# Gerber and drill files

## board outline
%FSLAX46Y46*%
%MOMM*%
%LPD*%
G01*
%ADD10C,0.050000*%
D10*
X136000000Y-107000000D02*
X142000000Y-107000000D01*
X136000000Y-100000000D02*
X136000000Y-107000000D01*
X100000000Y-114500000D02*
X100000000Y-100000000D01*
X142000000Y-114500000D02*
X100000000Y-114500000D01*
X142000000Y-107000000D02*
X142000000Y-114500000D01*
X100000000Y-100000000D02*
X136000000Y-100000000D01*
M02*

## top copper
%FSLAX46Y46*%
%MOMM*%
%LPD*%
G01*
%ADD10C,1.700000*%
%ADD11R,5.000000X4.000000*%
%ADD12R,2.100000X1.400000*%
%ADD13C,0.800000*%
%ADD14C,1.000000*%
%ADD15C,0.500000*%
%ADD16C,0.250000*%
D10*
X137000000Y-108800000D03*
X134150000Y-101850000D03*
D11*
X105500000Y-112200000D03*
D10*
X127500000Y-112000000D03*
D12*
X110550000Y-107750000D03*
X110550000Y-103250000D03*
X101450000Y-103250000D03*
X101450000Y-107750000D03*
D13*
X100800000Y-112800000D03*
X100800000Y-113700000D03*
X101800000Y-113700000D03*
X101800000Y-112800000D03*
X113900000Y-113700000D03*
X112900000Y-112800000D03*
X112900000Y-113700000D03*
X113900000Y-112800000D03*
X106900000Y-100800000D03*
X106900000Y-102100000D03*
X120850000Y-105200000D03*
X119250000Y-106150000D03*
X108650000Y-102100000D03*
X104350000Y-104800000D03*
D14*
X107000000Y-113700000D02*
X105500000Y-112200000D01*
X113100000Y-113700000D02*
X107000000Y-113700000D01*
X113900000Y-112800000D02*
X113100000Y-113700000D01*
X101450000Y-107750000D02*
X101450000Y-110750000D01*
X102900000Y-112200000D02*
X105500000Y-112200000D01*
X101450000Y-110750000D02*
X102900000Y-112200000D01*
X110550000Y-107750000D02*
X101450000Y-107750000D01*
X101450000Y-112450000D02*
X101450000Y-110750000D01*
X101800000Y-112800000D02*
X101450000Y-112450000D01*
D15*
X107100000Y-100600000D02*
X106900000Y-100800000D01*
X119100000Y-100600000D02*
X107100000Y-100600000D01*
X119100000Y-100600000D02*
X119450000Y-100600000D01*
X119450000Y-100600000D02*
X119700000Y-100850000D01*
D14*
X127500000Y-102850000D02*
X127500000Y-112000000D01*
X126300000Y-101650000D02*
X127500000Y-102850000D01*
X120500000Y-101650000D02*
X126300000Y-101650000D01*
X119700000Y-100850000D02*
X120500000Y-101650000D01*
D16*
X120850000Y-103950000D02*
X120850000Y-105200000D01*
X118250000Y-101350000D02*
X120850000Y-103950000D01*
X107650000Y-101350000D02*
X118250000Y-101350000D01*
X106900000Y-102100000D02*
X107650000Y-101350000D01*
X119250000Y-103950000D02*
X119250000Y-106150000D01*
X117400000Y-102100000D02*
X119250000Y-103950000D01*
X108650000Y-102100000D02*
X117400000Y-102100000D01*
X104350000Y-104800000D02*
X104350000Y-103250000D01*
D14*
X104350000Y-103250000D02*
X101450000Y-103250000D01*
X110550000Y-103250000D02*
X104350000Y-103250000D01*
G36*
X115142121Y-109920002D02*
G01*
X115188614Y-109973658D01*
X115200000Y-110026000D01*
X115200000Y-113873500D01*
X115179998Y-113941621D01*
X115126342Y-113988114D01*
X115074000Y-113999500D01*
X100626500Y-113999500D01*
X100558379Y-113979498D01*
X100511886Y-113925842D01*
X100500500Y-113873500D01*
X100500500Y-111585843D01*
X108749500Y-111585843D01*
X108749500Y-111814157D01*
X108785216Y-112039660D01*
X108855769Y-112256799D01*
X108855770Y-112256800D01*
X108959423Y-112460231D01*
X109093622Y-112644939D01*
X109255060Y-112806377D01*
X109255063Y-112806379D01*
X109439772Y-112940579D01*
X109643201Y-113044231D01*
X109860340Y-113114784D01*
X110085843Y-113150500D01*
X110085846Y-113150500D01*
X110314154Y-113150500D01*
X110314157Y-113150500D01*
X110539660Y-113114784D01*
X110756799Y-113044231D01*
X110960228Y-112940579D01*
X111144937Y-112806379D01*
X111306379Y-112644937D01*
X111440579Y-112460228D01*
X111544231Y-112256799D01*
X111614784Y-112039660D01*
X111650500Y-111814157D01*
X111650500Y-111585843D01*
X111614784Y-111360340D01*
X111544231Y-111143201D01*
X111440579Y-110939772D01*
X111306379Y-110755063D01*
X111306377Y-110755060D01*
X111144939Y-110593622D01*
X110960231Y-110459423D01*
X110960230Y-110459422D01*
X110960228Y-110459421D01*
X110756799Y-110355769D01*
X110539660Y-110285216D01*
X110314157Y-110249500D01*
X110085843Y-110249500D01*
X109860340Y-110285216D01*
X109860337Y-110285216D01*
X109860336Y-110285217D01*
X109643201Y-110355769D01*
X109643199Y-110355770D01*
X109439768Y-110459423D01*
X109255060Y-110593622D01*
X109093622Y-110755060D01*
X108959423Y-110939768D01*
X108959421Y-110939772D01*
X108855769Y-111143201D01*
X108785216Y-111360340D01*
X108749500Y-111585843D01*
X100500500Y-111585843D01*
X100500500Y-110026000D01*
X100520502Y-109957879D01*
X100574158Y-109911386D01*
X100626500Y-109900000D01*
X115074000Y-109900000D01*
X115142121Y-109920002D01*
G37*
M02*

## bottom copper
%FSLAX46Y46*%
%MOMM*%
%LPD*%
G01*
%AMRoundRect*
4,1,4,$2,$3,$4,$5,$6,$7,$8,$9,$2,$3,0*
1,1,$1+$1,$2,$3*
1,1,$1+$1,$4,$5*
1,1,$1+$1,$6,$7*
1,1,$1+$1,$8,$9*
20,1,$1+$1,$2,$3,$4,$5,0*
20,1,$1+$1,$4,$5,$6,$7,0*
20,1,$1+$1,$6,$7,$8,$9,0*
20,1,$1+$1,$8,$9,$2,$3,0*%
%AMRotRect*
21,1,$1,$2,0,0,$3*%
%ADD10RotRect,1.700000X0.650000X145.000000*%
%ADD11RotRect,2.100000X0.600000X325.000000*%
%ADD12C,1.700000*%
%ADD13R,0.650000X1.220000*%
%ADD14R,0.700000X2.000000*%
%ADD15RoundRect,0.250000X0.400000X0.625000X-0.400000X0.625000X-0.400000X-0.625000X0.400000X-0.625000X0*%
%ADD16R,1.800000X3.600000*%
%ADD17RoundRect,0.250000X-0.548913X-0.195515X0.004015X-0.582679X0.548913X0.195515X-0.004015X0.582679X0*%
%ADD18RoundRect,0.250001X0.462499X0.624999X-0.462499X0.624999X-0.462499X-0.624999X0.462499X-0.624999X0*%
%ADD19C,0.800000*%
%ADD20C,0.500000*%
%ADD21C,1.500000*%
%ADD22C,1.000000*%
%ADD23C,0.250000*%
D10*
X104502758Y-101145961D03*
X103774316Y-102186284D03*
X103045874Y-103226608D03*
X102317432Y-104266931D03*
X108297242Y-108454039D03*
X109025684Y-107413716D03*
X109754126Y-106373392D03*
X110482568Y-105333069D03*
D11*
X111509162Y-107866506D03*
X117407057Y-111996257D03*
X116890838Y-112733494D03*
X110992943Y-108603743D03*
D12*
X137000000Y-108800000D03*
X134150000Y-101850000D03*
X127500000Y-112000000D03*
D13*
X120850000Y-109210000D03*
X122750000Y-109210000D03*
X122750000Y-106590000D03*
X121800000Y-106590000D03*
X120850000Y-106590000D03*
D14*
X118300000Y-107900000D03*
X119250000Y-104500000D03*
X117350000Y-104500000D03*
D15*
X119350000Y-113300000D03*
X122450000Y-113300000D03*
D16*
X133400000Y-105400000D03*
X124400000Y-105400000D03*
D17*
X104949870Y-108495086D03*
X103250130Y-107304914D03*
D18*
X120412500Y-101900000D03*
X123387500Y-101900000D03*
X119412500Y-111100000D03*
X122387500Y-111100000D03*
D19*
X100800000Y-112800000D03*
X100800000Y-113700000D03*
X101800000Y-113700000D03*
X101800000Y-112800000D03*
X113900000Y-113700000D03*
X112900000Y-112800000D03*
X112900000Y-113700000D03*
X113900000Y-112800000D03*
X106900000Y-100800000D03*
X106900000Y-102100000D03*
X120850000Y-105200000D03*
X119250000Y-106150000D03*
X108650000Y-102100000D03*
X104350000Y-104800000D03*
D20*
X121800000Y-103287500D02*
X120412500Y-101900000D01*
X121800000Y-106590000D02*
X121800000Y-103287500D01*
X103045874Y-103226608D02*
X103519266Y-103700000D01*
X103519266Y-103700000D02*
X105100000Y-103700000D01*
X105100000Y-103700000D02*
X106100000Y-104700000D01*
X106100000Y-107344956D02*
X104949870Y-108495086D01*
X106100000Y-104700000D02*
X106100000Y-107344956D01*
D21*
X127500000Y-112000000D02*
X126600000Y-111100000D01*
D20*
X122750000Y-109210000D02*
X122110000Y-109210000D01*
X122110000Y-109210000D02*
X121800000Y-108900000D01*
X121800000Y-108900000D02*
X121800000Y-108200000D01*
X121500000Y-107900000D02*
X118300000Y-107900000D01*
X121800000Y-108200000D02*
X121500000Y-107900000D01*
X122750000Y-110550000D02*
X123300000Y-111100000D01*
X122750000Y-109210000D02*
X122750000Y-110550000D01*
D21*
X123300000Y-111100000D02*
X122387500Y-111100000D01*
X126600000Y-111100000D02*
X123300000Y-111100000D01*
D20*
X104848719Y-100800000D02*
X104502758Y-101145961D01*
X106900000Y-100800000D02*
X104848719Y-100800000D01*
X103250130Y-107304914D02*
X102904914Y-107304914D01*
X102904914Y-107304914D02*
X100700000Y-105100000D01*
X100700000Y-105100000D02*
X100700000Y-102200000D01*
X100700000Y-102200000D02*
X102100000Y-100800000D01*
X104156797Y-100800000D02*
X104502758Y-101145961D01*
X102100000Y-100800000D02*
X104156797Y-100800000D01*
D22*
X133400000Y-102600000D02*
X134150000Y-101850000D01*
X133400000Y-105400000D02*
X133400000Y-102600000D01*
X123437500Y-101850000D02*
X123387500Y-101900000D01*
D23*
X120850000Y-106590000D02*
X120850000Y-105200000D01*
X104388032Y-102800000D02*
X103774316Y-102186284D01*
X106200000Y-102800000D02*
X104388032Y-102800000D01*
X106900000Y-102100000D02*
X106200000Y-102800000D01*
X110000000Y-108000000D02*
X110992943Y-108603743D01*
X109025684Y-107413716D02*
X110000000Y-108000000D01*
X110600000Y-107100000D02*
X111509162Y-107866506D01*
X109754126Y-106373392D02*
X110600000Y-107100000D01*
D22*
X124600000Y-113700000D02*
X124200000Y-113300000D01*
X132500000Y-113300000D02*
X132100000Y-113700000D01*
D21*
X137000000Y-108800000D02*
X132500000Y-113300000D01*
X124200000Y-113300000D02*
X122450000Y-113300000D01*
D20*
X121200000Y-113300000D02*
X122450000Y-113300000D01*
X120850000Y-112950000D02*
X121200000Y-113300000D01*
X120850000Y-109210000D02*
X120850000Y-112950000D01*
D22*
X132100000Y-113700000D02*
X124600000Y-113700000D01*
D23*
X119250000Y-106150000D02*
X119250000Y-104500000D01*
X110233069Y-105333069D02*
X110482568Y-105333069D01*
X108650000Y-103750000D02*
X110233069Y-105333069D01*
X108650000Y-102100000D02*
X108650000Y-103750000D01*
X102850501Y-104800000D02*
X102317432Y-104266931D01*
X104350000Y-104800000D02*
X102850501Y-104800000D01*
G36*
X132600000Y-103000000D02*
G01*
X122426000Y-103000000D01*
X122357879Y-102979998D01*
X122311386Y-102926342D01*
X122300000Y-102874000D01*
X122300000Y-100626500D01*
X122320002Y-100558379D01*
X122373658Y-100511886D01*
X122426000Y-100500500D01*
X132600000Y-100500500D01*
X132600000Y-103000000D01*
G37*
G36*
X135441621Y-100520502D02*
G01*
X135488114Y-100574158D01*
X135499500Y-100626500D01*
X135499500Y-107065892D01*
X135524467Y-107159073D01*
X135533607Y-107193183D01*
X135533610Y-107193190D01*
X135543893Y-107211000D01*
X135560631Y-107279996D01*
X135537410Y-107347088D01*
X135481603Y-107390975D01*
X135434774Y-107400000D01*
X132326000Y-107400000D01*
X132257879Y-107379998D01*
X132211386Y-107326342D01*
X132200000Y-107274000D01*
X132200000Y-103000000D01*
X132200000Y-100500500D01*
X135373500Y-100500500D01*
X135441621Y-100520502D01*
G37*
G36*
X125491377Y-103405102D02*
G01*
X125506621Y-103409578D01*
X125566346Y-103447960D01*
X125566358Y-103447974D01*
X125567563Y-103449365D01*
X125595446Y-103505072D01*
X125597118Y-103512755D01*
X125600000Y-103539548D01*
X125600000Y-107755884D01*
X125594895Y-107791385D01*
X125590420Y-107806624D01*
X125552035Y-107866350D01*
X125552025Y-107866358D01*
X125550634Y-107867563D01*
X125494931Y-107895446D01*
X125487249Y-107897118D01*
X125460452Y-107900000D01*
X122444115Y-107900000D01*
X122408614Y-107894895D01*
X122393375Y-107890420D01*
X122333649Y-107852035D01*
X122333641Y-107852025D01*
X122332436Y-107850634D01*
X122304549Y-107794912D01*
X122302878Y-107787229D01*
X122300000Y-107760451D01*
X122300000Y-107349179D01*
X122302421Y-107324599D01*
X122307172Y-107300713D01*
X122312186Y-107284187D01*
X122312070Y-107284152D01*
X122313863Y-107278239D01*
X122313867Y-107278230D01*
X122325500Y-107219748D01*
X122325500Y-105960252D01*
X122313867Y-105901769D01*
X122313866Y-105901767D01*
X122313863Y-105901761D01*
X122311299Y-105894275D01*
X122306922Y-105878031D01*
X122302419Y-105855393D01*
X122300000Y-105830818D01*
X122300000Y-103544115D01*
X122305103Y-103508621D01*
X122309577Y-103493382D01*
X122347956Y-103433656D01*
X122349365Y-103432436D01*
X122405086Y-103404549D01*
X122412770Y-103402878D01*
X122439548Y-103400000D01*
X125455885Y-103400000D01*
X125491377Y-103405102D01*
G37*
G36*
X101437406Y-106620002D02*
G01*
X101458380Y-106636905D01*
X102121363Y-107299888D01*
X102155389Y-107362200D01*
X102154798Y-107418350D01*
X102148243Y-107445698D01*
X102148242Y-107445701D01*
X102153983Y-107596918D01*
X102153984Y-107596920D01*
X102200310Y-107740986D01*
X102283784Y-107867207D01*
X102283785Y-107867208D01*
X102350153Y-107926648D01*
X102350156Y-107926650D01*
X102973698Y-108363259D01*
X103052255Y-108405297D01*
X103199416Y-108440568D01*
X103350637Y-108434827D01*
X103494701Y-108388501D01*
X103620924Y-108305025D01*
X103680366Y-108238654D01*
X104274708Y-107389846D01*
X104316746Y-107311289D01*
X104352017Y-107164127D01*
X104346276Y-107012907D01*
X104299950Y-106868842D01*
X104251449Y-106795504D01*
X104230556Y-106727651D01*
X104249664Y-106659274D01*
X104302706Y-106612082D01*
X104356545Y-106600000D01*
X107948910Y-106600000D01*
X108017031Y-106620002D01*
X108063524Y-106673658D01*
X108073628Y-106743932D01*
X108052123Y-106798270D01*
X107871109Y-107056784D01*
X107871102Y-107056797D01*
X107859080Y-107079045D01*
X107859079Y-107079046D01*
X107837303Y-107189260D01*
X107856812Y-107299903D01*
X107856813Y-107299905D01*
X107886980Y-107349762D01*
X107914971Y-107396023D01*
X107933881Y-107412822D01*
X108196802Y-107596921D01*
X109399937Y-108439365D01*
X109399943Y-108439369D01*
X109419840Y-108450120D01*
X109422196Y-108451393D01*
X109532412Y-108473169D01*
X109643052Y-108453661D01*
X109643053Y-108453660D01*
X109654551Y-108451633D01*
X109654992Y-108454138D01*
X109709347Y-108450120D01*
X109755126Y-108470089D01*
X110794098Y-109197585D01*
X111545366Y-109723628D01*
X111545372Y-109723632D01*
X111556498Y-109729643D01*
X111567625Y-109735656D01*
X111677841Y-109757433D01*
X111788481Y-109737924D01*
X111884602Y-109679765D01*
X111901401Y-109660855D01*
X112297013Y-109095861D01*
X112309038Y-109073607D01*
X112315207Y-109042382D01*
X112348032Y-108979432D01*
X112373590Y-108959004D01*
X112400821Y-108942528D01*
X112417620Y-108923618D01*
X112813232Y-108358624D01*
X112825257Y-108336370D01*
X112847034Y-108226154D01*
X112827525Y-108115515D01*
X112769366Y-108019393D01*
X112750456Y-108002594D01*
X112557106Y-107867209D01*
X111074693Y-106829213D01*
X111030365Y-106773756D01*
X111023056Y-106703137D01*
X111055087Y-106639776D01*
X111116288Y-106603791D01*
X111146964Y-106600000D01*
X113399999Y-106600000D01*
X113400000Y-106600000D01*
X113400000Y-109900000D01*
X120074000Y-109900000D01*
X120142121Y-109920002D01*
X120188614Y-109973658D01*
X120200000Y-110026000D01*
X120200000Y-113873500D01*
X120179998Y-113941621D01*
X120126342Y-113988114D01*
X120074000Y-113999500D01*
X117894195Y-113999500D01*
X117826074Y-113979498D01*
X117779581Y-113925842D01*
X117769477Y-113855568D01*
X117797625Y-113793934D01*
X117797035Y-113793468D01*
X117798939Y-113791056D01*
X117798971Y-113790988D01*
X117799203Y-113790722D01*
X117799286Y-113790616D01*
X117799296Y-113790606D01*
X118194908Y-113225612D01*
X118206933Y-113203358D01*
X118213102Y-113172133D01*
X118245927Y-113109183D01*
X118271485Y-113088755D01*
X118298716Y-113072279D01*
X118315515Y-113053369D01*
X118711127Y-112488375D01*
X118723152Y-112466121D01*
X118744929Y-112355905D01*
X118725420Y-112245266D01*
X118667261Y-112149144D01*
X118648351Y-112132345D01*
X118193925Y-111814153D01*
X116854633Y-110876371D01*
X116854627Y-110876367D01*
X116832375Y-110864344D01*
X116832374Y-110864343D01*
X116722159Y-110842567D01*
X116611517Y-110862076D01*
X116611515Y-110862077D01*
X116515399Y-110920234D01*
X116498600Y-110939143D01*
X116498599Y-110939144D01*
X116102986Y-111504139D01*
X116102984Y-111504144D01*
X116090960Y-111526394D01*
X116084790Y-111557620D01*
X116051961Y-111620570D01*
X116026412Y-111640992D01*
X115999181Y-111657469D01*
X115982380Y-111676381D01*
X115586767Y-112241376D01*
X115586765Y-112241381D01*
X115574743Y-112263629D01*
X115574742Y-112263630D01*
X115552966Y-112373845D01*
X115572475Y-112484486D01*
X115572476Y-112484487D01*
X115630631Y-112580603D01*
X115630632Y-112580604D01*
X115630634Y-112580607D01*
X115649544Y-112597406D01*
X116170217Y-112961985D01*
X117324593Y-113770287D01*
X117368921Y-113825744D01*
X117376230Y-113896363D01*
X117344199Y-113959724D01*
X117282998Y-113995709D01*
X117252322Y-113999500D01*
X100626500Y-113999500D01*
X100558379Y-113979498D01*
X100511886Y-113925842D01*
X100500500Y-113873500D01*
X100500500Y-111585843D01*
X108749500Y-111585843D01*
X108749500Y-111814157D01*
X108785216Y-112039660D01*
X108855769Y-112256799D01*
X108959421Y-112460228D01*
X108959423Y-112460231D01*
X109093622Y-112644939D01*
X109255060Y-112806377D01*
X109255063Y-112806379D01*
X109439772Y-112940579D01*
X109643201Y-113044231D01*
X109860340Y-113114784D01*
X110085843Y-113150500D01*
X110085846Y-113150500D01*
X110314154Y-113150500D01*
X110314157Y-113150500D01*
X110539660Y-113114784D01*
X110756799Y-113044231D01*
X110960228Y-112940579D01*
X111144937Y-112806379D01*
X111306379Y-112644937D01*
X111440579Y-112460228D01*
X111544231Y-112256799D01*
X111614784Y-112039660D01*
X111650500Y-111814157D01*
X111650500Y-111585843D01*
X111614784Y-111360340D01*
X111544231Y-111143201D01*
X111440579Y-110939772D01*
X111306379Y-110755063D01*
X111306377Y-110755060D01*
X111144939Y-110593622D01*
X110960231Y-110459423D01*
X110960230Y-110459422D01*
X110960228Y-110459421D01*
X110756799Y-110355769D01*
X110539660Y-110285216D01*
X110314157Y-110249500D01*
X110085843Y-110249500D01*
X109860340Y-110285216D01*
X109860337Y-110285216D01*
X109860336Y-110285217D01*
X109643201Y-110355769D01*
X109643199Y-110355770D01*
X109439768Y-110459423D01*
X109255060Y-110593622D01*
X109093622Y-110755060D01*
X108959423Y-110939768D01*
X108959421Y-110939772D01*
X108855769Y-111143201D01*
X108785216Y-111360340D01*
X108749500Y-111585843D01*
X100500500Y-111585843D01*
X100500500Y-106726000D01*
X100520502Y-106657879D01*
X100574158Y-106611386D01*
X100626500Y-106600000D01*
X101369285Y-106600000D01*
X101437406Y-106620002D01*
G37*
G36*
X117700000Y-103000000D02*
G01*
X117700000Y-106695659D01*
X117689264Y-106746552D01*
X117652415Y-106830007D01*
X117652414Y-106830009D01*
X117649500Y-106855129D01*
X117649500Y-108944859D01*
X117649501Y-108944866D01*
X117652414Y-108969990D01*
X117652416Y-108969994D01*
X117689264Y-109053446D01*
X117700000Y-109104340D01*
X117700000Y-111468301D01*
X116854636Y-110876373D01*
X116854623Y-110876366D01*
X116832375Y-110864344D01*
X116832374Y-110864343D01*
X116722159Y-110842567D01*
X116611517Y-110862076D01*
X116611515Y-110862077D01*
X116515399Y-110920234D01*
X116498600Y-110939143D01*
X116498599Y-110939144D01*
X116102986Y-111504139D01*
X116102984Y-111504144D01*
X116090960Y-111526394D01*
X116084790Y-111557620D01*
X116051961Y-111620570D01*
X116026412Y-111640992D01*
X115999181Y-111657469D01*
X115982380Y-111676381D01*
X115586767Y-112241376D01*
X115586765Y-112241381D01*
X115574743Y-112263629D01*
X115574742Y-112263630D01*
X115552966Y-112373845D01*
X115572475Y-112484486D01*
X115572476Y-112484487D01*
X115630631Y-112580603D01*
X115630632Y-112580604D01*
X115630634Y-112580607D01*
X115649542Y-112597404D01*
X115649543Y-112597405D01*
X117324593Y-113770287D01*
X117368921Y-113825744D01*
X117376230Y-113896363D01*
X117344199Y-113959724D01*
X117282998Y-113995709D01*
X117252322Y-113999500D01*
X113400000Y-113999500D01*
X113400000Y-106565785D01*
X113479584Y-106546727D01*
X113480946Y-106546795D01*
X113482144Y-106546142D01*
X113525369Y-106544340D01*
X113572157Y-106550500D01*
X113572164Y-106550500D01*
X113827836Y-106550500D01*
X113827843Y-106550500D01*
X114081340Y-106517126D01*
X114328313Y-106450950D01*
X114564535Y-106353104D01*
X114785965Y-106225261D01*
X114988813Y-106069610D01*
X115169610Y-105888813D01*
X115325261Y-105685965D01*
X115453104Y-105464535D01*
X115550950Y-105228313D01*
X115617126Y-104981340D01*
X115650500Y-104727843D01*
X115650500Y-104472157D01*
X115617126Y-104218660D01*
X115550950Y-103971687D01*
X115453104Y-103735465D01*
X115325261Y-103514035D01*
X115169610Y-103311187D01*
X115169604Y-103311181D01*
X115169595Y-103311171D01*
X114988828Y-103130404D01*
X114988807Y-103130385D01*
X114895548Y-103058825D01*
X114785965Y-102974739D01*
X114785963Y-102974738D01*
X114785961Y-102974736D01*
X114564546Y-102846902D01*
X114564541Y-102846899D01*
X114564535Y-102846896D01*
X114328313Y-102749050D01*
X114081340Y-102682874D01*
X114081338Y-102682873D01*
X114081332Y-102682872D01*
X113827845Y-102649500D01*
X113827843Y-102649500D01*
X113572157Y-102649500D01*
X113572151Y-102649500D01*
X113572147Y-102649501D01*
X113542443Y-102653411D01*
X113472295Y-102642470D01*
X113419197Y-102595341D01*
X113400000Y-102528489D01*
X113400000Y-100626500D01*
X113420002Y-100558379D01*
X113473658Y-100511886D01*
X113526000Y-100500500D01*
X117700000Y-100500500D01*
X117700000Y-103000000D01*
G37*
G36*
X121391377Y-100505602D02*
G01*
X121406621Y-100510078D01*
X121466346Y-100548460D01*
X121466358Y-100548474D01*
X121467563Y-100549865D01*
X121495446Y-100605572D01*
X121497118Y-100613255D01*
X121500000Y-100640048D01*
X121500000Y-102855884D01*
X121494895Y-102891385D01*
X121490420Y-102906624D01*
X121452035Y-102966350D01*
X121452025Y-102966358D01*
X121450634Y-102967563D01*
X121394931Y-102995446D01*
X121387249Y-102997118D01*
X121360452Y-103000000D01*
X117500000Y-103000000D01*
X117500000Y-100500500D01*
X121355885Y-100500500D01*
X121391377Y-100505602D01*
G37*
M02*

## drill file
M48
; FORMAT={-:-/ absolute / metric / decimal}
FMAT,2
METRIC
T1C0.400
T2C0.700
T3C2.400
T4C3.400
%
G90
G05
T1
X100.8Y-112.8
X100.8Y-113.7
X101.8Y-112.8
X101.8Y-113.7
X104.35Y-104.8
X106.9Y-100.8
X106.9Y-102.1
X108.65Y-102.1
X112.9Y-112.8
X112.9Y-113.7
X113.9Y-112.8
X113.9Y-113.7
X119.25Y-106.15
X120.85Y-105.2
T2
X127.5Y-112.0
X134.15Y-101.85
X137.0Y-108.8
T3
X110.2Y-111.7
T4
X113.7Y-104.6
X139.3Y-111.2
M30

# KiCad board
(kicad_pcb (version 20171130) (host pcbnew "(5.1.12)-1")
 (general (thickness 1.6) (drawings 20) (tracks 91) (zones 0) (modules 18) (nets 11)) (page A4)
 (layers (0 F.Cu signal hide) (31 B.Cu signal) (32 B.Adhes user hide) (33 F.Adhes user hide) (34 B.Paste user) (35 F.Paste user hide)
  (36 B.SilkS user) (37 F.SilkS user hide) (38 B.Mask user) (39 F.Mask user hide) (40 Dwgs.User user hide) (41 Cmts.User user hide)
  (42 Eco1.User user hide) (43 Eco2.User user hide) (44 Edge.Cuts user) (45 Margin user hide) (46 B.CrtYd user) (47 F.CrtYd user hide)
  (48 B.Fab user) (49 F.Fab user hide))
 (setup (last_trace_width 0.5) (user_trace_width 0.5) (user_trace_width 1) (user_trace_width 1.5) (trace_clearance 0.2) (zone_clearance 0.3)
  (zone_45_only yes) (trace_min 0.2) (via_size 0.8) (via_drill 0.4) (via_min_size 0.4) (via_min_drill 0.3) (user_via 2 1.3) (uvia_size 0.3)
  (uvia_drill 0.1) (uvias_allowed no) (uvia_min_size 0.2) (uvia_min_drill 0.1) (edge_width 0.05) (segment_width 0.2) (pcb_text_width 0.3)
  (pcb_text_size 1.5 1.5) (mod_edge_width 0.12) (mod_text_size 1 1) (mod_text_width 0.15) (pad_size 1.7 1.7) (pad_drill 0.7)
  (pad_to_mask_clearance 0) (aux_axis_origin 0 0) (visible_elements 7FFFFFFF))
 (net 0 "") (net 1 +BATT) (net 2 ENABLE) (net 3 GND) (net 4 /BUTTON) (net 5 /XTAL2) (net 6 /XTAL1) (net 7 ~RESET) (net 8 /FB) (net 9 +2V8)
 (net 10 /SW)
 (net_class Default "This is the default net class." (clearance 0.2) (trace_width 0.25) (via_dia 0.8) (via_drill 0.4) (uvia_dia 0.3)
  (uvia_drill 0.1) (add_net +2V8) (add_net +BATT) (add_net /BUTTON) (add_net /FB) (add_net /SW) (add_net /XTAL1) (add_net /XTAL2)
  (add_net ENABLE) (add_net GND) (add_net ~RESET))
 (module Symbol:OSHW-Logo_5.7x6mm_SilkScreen (layer F.Cu) (at 132.1 106.2)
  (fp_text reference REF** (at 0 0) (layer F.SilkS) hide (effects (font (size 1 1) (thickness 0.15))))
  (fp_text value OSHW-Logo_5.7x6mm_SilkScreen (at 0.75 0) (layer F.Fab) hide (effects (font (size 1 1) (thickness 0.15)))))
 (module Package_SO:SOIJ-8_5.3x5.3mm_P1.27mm (layer B.Cu) (at 106.4 104.8 145)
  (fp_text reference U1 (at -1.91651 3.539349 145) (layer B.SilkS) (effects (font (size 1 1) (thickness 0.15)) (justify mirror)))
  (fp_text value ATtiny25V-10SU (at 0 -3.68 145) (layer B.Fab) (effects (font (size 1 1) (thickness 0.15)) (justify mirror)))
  (pad 8 smd rect (at 3.65 1.905 145) (size 1.7 0.65) (layers B.Cu B.Paste B.Mask) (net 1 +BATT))
  (pad 7 smd rect (at 3.65 0.635 145) (size 1.7 0.65) (layers B.Cu B.Paste B.Mask) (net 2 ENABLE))
  (pad 6 smd rect (at 3.65 -0.635 145) (size 1.7 0.65) (layers B.Cu B.Paste B.Mask) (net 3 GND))
  (pad 5 smd rect (at 3.65 -1.905 145) (size 1.7 0.65) (layers B.Cu B.Paste B.Mask) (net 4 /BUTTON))
  (pad 4 smd rect (at -3.65 -1.905 145) (size 1.7 0.65) (layers B.Cu B.Paste B.Mask) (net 3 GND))
  (pad 3 smd rect (at -3.65 -0.635 145) (size 1.7 0.65) (layers B.Cu B.Paste B.Mask) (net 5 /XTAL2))
  (pad 2 smd rect (at -3.65 0.635 145) (size 1.7 0.65) (layers B.Cu B.Paste B.Mask) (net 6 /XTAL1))
  (pad 1 smd rect (at -3.65 1.905 145) (size 1.7 0.65) (layers B.Cu B.Paste B.Mask) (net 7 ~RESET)))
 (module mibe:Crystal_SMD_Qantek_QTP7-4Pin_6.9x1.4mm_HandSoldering (layer B.Cu) (at 114.2 110.3 325)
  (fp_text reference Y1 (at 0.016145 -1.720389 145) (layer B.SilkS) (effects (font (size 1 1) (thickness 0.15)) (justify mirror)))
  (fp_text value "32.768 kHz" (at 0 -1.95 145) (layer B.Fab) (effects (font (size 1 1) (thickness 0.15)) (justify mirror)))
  (pad 1 smd rect (at -3.6 -0.45 325) (size 2.1 0.6) (layers B.Cu B.Paste B.Mask) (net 6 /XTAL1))
  (pad NC smd rect (at 3.6 -0.45 325) (size 2.1 0.6) (layers B.Cu B.Paste B.Mask))
  (pad NC smd rect (at 3.6 0.45 325) (size 2.1 0.6) (layers B.Cu B.Paste B.Mask))
  (pad 2 smd rect (at -3.6 0.45 325) (size 2.1 0.6) (layers B.Cu B.Paste B.Mask) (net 5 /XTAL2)))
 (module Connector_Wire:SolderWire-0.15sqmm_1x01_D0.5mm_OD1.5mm (layer F.Cu) (at 137 108.8)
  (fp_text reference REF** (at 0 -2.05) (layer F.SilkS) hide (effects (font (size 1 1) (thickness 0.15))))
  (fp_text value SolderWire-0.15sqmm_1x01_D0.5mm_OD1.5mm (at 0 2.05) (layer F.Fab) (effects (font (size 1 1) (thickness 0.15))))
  (pad 1 thru_hole circle (at 0 0) (size 1.7 1.7) (drill 0.7) (layers *.Cu *.Mask) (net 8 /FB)))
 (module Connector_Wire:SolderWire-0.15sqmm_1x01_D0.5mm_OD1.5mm (layer F.Cu) (at 134.15 101.85)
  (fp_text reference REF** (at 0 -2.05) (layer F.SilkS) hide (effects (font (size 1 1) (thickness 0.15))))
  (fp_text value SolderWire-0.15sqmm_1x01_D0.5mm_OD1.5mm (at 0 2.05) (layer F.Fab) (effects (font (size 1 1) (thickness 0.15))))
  (pad 1 thru_hole circle (at 0 0) (size 1.7 1.7) (drill 0.7) (layers *.Cu *.Mask) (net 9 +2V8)))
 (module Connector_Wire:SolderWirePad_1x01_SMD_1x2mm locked (layer F.Cu) (at 105.5 112.2)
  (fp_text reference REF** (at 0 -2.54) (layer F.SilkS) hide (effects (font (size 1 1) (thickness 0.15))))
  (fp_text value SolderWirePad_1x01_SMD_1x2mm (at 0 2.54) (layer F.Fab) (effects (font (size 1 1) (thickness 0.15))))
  (pad 1 smd rect (at 0 0) (size 5 4) (layers F.Cu F.Paste F.Mask) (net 3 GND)))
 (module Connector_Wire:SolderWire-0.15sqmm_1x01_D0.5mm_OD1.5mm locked (layer F.Cu) (at 127.5 112)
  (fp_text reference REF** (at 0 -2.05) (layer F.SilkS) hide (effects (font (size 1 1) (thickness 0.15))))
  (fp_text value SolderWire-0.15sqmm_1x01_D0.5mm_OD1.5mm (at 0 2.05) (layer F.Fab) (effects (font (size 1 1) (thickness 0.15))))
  (pad 1 thru_hole circle (at 0 0) (size 1.7 1.7) (drill 0.7) (layers *.Cu *.Mask) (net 1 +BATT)))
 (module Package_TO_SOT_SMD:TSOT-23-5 (layer B.Cu) (at 121.8 107.9 270)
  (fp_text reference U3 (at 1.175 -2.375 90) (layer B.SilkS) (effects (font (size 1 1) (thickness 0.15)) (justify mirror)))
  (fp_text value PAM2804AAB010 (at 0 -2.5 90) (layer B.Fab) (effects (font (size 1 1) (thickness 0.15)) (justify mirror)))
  (pad 5 smd rect (at 1.31 0.95 270) (size 1.22 0.65) (layers B.Cu B.Paste B.Mask) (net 8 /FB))
  (pad 4 smd rect (at 1.31 -0.95 270) (size 1.22 0.65) (layers B.Cu B.Paste B.Mask) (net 1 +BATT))
  (pad 3 smd rect (at -1.31 -0.95 270) (size 1.22 0.65) (layers B.Cu B.Paste B.Mask) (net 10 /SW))
  (pad 2 smd rect (at -1.31 0 270) (size 1.22 0.65) (layers B.Cu B.Paste B.Mask) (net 3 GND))
  (pad 1 smd rect (at -1.31 0.95 270) (size 1.22 0.65) (layers B.Cu B.Paste B.Mask) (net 2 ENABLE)))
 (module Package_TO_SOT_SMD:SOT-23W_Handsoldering (layer B.Cu) (at 118.3 106.2 270)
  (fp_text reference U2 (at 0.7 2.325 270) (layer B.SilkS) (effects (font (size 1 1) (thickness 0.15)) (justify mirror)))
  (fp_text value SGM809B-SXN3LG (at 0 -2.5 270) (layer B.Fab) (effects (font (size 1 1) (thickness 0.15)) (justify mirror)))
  (pad 3 smd rect (at 1.7 0 270) (size 2 0.7) (layers B.Cu B.Paste B.Mask) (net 1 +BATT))
  (pad 2 smd rect (at -1.7 -0.95 270) (size 2 0.7) (layers B.Cu B.Paste B.Mask) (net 7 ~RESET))
  (pad 1 smd rect (at -1.7 0.95 270) (size 2 0.7) (layers B.Cu B.Paste B.Mask) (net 3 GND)))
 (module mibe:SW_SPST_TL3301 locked (layer F.Cu) (at 106 105.5)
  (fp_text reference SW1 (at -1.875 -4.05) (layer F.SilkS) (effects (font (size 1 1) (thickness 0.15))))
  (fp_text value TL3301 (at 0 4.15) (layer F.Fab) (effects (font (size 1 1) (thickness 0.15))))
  (pad 2 smd rect (at 4.55 2.25) (size 2.1 1.4) (layers F.Cu F.Paste F.Mask) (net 3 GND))
  (pad 1 smd rect (at 4.55 -2.25) (size 2.1 1.4) (layers F.Cu F.Paste F.Mask) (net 4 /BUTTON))
  (pad 1 smd rect (at -4.55 -2.25) (size 2.1 1.4) (layers F.Cu F.Paste F.Mask) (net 4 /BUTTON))
  (pad 2 smd rect (at -4.55 2.25) (size 2.1 1.4) (layers F.Cu F.Paste F.Mask) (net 3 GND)))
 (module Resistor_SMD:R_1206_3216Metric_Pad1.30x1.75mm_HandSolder (layer B.Cu) (at 120.9 113.3 180)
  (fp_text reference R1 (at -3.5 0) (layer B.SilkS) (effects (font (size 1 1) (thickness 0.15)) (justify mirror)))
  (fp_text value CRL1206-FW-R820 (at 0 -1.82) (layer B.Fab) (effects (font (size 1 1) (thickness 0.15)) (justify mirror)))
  (pad 2 smd roundrect (at 1.55 0 180) (size 1.3 1.75) (layers B.Cu B.Paste B.Mask) (roundrect_rratio 0.192308) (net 3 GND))
  (pad 1 smd roundrect (at -1.55 0 180) (size 1.3 1.75) (layers B.Cu B.Paste B.Mask) (roundrect_rratio 0.192308) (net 8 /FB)))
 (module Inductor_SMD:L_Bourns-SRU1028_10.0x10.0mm (layer B.Cu) (at 128.9 105.4)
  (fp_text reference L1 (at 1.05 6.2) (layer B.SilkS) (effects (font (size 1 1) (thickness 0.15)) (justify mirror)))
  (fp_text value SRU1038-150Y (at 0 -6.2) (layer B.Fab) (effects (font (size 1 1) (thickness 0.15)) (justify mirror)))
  (pad 2 smd rect (at 4.5 0) (size 1.8 3.6) (layers B.Cu B.Paste B.Mask) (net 9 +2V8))
  (pad 1 smd rect (at -4.5 0) (size 1.8 3.6) (layers B.Cu B.Paste B.Mask) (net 10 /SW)))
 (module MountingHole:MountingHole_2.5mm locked (layer F.Cu) (at 110.2 111.7)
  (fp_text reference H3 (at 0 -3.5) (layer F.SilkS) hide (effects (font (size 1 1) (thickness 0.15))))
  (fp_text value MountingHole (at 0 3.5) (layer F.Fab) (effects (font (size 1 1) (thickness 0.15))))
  (pad "" np_thru_hole circle (at 0 0) (size 2.4 2.4) (drill 2.4) (layers *.Cu *.Mask)))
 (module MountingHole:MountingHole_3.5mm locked (layer F.Cu) (at 139.3 111.2)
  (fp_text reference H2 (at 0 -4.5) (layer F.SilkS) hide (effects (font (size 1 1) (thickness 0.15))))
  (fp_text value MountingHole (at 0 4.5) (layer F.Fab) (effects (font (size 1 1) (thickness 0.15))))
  (pad "" np_thru_hole circle (at 0 0) (size 3.4 3.4) (drill 3.4) (layers *.Cu *.Mask)))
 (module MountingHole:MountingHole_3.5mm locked (layer F.Cu) (at 113.7 104.6)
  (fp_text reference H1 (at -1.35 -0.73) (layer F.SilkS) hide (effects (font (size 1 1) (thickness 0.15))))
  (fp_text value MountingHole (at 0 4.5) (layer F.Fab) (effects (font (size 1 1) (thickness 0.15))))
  (pad "" np_thru_hole circle (at 0 0) (size 3.4 3.4) (drill 3.4) (layers *.Cu *.Mask)))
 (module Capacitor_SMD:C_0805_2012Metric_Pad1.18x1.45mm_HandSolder (layer B.Cu) (at 104.1 107.9 325)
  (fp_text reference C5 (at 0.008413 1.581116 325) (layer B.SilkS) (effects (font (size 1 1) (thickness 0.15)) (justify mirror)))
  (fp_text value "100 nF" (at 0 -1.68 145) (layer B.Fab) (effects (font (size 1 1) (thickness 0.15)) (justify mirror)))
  (pad 2 smd roundrect (at 1.0375 0 325) (size 1.175 1.45) (layers B.Cu B.Paste B.Mask) (roundrect_rratio 0.212766) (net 3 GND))
  (pad 1 smd roundrect (at -1.0375 0 325) (size 1.175 1.45) (layers B.Cu B.Paste B.Mask) (roundrect_rratio 0.212766) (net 1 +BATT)))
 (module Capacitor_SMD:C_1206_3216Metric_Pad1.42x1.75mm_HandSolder (layer B.Cu) (at 121.9 101.9 180)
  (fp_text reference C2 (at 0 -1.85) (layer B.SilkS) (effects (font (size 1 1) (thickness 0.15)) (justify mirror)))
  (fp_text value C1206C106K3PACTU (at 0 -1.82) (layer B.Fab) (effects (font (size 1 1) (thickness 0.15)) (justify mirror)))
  (pad 2 smd roundrect (at 1.4875 0 180) (size 1.425 1.75) (layers B.Cu B.Paste B.Mask) (roundrect_rratio 0.175439) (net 3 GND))
  (pad 1 smd roundrect (at -1.4875 0 180) (size 1.425 1.75) (layers B.Cu B.Paste B.Mask) (roundrect_rratio 0.175439) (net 9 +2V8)))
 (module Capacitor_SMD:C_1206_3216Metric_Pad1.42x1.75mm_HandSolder (layer B.Cu) (at 120.9 111.1 180)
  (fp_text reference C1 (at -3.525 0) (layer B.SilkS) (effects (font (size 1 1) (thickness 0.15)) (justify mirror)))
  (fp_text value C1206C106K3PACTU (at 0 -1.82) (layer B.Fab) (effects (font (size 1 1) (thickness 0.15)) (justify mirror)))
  (pad 2 smd roundrect (at 1.4875 0 180) (size 1.425 1.75) (layers B.Cu B.Paste B.Mask) (roundrect_rratio 0.175439) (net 3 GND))
  (pad 1 smd roundrect (at -1.4875 0 180) (size 1.425 1.75) (layers B.Cu B.Paste B.Mask) (roundrect_rratio 0.175439) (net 1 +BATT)))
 (gr_line (start 136 107) (end 142 107) (layer Edge.Cuts) (width 0.05))
 (gr_line (start 136 100) (end 136 107) (layer Edge.Cuts) (width 0.05))
 (gr_line (start 100 114.5) (end 100 100) (layer Edge.Cuts) (width 0.05))
 (gr_line (start 142 114.5) (end 100 114.5) (layer Edge.Cuts) (width 0.05))
 (gr_line (start 142 107) (end 142 114.5) (layer Edge.Cuts) (width 0.05))
 (gr_line (start 100 100) (end 136 100) (layer Edge.Cuts) (width 0.05))
 (via (at 100.8 112.8) (size 0.8) (drill 0.4) (layers F.Cu B.Cu) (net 3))
 (via (at 100.8 113.7) (size 0.8) (drill 0.4) (layers F.Cu B.Cu) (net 3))
 (via (at 101.8 113.7) (size 0.8) (drill 0.4) (layers F.Cu B.Cu) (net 3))
 (via (at 101.8 112.8) (size 0.8) (drill 0.4) (layers F.Cu B.Cu) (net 3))
 (via (at 113.9 113.7) (size 0.8) (drill 0.4) (layers F.Cu B.Cu) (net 3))
 (via (at 112.9 112.8) (size 0.8) (drill 0.4) (layers F.Cu B.Cu) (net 3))
 (via (at 112.9 113.7) (size 0.8) (drill 0.4) (layers F.Cu B.Cu) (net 3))
 (via (at 113.9 112.8) (size 0.8) (drill 0.4) (layers F.Cu B.Cu) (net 3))
 (segment (start 107 113.7) (end 105.5 112.2) (width 1) (layer F.Cu) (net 3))
 (segment (start 113.1 113.7) (end 107 113.7) (width 1) (layer F.Cu) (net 3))
 (segment (start 113.9 112.8) (end 113.1 113.7) (width 1) (layer F.Cu) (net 3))
 (segment (start 101.45 107.75) (end 101.45 110.75) (width 1) (layer F.Cu) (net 3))
 (segment (start 102.9 112.2) (end 105.5 112.2) (width 1) (layer F.Cu) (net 3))
 (segment (start 101.45 110.75) (end 102.9 112.2) (width 1) (layer F.Cu) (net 3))
 (segment (start 110.55 107.75) (end 101.45 107.75) (width 1) (layer F.Cu) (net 3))
 (segment (start 121.8 103.2875) (end 120.4125 101.9) (width 0.5) (layer B.Cu) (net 3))
 (segment (start 121.8 106.59) (end 121.8 103.2875) (width 0.5) (layer B.Cu) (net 3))
 (segment (start 101.45 112.45) (end 101.45 110.75) (width 1) (layer F.Cu) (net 3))
 (segment (start 101.8 112.8) (end 101.45 112.45) (width 1) (layer F.Cu) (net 3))
 (segment (start 103.045874 103.226608) (end 103.519266 103.7) (width 0.5) (layer B.Cu) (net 3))
 (segment (start 103.519266 103.7) (end 105.1 103.7) (width 0.5) (layer B.Cu) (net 3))
 (segment (start 105.1 103.7) (end 106.1 104.7) (width 0.5) (layer B.Cu) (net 3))
 (segment (start 106.1 107.344956) (end 104.94987 108.495086) (width 0.5) (layer B.Cu) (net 3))
 (segment (start 106.1 104.7) (end 106.1 107.344956) (width 0.5) (layer B.Cu) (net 3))
 (via (at 106.9 100.8) (size 0.8) (drill 0.4) (layers F.Cu B.Cu) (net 1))
 (segment (start 127.5 112) (end 126.6 111.1) (width 1.5) (layer B.Cu) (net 1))
 (segment (start 122.75 109.21) (end 122.11 109.21) (width 0.5) (layer B.Cu) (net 1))
 (segment (start 122.11 109.21) (end 121.8 108.9) (width 0.5) (layer B.Cu) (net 1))
 (segment (start 121.8 108.9) (end 121.8 108.2) (width 0.5) (layer B.Cu) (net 1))
 (segment (start 121.5 107.9) (end 118.3 107.9) (width 0.5) (layer B.Cu) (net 1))
 (segment (start 121.8 108.2) (end 121.5 107.9) (width 0.5) (layer B.Cu) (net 1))
 (segment (start 122.75 110.55) (end 123.3 111.1) (width 0.5) (layer B.Cu) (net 1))
 (segment (start 122.75 109.21) (end 122.75 110.55) (width 0.5) (layer B.Cu) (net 1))
 (segment (start 123.3 111.1) (end 122.3875 111.1) (width 1.5) (layer B.Cu) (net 1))
 (segment (start 126.6 111.1) (end 123.3 111.1) (width 1.5) (layer B.Cu) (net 1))
 (segment (start 107.1 100.6) (end 106.9 100.8) (width 0.5) (layer F.Cu) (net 1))
 (segment (start 119.1 100.6) (end 107.1 100.6) (width 0.5) (layer F.Cu) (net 1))
 (segment (start 119.1 100.6) (end 119.45 100.6) (width 0.5) (layer F.Cu) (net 1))
 (segment (start 119.45 100.6) (end 119.7 100.85) (width 0.5) (layer F.Cu) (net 1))
 (segment (start 127.5 102.85) (end 127.5 112) (width 1) (layer F.Cu) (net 1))
 (segment (start 126.3 101.65) (end 127.5 102.85) (width 1) (layer F.Cu) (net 1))
 (segment (start 120.5 101.65) (end 126.3 101.65) (width 1) (layer F.Cu) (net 1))
 (segment (start 119.7 100.85) (end 120.5 101.65) (width 1) (layer F.Cu) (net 1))
 (segment (start 104.848719 100.8) (end 104.502758 101.145961) (width 0.5) (layer B.Cu) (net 1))
 (segment (start 106.9 100.8) (end 104.848719 100.8) (width 0.5) (layer B.Cu) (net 1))
 (segment (start 103.25013 107.304914) (end 102.904914 107.304914) (width 0.5) (layer B.Cu) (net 1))
 (segment (start 102.904914 107.304914) (end 100.7 105.1) (width 0.5) (layer B.Cu) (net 1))
 (segment (start 100.7 105.1) (end 100.7 102.2) (width 0.5) (layer B.Cu) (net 1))
 (segment (start 100.7 102.2) (end 102.1 100.8) (width 0.5) (layer B.Cu) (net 1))
 (segment (start 104.156797 100.8) (end 104.502758 101.145961) (width 0.5) (layer B.Cu) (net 1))
 (segment (start 102.1 100.8) (end 104.156797 100.8) (width 0.5) (layer B.Cu) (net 1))
 (segment (start 133.4 102.6) (end 134.15 101.85) (width 1) (layer B.Cu) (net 9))
 (segment (start 133.4 105.4) (end 133.4 102.6) (width 1) (layer B.Cu) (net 9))
 (segment (start 123.4375 101.85) (end 123.3875 101.9) (width 1) (layer B.Cu) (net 9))
 (via (at 106.9 102.1) (size 0.8) (drill 0.4) (layers F.Cu B.Cu) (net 2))
 (segment (start 120.85 106.59) (end 120.85 105.2) (width 0.25) (layer B.Cu) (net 2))
 (via (at 120.85 105.2) (size 0.8) (drill 0.4) (layers F.Cu B.Cu) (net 2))
 (segment (start 120.85 103.95) (end 120.85 105.2) (width 0.25) (layer F.Cu) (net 2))
 (segment (start 118.25 101.35) (end 120.85 103.95) (width 0.25) (layer F.Cu) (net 2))
 (segment (start 107.65 101.35) (end 118.25 101.35) (width 0.25) (layer F.Cu) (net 2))
 (segment (start 106.9 102.1) (end 107.65 101.35) (width 0.25) (layer F.Cu) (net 2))
 (segment (start 104.388032 102.8) (end 103.774316 102.186284) (width 0.25) (layer B.Cu) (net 2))
 (segment (start 106.2 102.8) (end 104.388032 102.8) (width 0.25) (layer B.Cu) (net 2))
 (segment (start 106.9 102.1) (end 106.2 102.8) (width 0.25) (layer B.Cu) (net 2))
 (segment (start 110 108) (end 110.992943 108.603743) (width 0.25) (layer B.Cu) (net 5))
 (segment (start 109.025684 107.413716) (end 110 108) (width 0.25) (layer B.Cu) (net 5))
 (segment (start 110.6 107.1) (end 111.509162 107.866506) (width 0.25) (layer B.Cu) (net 6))
 (segment (start 109.754126 106.373392) (end 110.6 107.1) (width 0.25) (layer B.Cu) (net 6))
 (segment (start 124.6 113.7) (end 124.2 113.3) (width 1) (layer B.Cu) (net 8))
 (segment (start 132.5 113.3) (end 132.1 113.7) (width 1) (layer B.Cu) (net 8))
 (segment (start 137 108.8) (end 132.5 113.3) (width 1.5) (layer B.Cu) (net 8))
 (segment (start 124.2 113.3) (end 122.45 113.3) (width 1.5) (layer B.Cu) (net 8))
 (segment (start 121.2 113.3) (end 122.45 113.3) (width 0.5) (layer B.Cu) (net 8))
 (segment (start 120.85 112.95) (end 121.2 113.3) (width 0.5) (layer B.Cu) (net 8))
 (segment (start 120.85 109.21) (end 120.85 112.95) (width 0.5) (layer B.Cu) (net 8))
 (segment (start 132.1 113.7) (end 124.6 113.7) (width 1) (layer B.Cu) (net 8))
 (via (at 119.25 106.15) (size 0.8) (drill 0.4) (layers F.Cu B.Cu) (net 7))
 (via (at 108.65 102.1) (size 0.8) (drill 0.4) (layers F.Cu B.Cu) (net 7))
 (segment (start 119.25 103.95) (end 119.25 106.15) (width 0.25) (layer F.Cu) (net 7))
 (segment (start 117.4 102.1) (end 119.25 103.95) (width 0.25) (layer F.Cu) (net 7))
 (segment (start 108.65 102.1) (end 117.4 102.1) (width 0.25) (layer F.Cu) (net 7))
 (segment (start 119.25 106.15) (end 119.25 104.5) (width 0.25) (layer B.Cu) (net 7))
 (segment (start 110.233069 105.333069) (end 110.482568 105.333069) (width 0.25) (layer B.Cu) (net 7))
 (segment (start 108.65 103.75) (end 110.233069 105.333069) (width 0.25) (layer B.Cu) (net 7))
 (segment (start 108.65 102.1) (end 108.65 103.75) (width 0.25) (layer B.Cu) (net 7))
 (via (at 104.35 104.8) (size 0.8) (drill 0.4) (layers F.Cu B.Cu) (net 4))
 (segment (start 104.35 104.8) (end 104.35 103.25) (width 0.25) (layer F.Cu) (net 4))
 (segment (start 104.35 103.25) (end 101.45 103.25) (width 1) (layer F.Cu) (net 4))
 (segment (start 110.55 103.25) (end 104.35 103.25) (width 1) (layer F.Cu) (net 4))
 (segment (start 102.850501 104.8) (end 102.317432 104.266931) (width 0.25) (layer B.Cu) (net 4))
 (segment (start 104.35 104.8) (end 102.850501 104.8) (width 0.25) (layer B.Cu) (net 4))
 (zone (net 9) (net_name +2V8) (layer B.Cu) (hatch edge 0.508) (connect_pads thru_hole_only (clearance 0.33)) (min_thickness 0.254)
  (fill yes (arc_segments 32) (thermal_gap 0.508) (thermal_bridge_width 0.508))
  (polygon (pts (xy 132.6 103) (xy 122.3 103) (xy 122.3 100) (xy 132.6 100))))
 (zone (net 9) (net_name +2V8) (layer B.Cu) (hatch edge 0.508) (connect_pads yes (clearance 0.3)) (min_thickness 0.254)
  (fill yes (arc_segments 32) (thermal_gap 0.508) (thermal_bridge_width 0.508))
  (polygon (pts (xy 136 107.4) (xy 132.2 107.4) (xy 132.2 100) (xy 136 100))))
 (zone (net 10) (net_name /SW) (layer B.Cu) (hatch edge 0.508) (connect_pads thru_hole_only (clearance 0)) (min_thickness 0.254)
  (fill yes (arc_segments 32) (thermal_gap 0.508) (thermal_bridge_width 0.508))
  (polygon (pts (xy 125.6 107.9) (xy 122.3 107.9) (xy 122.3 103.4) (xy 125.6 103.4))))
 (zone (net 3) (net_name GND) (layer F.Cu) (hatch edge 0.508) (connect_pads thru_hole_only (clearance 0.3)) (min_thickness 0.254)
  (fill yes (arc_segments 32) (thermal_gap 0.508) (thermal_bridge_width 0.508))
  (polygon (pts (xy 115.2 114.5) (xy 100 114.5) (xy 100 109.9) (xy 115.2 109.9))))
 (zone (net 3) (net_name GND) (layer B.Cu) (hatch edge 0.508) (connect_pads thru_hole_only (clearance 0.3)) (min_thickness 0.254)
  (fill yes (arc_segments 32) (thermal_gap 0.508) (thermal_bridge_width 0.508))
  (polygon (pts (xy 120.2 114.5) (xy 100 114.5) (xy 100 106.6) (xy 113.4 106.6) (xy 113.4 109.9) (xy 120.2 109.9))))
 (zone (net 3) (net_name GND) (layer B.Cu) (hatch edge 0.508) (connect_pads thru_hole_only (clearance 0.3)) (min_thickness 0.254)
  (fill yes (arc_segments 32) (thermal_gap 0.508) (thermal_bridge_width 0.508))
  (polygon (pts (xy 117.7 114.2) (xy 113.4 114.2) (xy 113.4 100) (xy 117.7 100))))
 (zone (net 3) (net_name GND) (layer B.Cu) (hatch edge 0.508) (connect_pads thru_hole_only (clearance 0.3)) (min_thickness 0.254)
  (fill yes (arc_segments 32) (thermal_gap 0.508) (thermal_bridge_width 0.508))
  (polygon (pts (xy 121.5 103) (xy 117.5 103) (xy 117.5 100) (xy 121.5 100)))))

